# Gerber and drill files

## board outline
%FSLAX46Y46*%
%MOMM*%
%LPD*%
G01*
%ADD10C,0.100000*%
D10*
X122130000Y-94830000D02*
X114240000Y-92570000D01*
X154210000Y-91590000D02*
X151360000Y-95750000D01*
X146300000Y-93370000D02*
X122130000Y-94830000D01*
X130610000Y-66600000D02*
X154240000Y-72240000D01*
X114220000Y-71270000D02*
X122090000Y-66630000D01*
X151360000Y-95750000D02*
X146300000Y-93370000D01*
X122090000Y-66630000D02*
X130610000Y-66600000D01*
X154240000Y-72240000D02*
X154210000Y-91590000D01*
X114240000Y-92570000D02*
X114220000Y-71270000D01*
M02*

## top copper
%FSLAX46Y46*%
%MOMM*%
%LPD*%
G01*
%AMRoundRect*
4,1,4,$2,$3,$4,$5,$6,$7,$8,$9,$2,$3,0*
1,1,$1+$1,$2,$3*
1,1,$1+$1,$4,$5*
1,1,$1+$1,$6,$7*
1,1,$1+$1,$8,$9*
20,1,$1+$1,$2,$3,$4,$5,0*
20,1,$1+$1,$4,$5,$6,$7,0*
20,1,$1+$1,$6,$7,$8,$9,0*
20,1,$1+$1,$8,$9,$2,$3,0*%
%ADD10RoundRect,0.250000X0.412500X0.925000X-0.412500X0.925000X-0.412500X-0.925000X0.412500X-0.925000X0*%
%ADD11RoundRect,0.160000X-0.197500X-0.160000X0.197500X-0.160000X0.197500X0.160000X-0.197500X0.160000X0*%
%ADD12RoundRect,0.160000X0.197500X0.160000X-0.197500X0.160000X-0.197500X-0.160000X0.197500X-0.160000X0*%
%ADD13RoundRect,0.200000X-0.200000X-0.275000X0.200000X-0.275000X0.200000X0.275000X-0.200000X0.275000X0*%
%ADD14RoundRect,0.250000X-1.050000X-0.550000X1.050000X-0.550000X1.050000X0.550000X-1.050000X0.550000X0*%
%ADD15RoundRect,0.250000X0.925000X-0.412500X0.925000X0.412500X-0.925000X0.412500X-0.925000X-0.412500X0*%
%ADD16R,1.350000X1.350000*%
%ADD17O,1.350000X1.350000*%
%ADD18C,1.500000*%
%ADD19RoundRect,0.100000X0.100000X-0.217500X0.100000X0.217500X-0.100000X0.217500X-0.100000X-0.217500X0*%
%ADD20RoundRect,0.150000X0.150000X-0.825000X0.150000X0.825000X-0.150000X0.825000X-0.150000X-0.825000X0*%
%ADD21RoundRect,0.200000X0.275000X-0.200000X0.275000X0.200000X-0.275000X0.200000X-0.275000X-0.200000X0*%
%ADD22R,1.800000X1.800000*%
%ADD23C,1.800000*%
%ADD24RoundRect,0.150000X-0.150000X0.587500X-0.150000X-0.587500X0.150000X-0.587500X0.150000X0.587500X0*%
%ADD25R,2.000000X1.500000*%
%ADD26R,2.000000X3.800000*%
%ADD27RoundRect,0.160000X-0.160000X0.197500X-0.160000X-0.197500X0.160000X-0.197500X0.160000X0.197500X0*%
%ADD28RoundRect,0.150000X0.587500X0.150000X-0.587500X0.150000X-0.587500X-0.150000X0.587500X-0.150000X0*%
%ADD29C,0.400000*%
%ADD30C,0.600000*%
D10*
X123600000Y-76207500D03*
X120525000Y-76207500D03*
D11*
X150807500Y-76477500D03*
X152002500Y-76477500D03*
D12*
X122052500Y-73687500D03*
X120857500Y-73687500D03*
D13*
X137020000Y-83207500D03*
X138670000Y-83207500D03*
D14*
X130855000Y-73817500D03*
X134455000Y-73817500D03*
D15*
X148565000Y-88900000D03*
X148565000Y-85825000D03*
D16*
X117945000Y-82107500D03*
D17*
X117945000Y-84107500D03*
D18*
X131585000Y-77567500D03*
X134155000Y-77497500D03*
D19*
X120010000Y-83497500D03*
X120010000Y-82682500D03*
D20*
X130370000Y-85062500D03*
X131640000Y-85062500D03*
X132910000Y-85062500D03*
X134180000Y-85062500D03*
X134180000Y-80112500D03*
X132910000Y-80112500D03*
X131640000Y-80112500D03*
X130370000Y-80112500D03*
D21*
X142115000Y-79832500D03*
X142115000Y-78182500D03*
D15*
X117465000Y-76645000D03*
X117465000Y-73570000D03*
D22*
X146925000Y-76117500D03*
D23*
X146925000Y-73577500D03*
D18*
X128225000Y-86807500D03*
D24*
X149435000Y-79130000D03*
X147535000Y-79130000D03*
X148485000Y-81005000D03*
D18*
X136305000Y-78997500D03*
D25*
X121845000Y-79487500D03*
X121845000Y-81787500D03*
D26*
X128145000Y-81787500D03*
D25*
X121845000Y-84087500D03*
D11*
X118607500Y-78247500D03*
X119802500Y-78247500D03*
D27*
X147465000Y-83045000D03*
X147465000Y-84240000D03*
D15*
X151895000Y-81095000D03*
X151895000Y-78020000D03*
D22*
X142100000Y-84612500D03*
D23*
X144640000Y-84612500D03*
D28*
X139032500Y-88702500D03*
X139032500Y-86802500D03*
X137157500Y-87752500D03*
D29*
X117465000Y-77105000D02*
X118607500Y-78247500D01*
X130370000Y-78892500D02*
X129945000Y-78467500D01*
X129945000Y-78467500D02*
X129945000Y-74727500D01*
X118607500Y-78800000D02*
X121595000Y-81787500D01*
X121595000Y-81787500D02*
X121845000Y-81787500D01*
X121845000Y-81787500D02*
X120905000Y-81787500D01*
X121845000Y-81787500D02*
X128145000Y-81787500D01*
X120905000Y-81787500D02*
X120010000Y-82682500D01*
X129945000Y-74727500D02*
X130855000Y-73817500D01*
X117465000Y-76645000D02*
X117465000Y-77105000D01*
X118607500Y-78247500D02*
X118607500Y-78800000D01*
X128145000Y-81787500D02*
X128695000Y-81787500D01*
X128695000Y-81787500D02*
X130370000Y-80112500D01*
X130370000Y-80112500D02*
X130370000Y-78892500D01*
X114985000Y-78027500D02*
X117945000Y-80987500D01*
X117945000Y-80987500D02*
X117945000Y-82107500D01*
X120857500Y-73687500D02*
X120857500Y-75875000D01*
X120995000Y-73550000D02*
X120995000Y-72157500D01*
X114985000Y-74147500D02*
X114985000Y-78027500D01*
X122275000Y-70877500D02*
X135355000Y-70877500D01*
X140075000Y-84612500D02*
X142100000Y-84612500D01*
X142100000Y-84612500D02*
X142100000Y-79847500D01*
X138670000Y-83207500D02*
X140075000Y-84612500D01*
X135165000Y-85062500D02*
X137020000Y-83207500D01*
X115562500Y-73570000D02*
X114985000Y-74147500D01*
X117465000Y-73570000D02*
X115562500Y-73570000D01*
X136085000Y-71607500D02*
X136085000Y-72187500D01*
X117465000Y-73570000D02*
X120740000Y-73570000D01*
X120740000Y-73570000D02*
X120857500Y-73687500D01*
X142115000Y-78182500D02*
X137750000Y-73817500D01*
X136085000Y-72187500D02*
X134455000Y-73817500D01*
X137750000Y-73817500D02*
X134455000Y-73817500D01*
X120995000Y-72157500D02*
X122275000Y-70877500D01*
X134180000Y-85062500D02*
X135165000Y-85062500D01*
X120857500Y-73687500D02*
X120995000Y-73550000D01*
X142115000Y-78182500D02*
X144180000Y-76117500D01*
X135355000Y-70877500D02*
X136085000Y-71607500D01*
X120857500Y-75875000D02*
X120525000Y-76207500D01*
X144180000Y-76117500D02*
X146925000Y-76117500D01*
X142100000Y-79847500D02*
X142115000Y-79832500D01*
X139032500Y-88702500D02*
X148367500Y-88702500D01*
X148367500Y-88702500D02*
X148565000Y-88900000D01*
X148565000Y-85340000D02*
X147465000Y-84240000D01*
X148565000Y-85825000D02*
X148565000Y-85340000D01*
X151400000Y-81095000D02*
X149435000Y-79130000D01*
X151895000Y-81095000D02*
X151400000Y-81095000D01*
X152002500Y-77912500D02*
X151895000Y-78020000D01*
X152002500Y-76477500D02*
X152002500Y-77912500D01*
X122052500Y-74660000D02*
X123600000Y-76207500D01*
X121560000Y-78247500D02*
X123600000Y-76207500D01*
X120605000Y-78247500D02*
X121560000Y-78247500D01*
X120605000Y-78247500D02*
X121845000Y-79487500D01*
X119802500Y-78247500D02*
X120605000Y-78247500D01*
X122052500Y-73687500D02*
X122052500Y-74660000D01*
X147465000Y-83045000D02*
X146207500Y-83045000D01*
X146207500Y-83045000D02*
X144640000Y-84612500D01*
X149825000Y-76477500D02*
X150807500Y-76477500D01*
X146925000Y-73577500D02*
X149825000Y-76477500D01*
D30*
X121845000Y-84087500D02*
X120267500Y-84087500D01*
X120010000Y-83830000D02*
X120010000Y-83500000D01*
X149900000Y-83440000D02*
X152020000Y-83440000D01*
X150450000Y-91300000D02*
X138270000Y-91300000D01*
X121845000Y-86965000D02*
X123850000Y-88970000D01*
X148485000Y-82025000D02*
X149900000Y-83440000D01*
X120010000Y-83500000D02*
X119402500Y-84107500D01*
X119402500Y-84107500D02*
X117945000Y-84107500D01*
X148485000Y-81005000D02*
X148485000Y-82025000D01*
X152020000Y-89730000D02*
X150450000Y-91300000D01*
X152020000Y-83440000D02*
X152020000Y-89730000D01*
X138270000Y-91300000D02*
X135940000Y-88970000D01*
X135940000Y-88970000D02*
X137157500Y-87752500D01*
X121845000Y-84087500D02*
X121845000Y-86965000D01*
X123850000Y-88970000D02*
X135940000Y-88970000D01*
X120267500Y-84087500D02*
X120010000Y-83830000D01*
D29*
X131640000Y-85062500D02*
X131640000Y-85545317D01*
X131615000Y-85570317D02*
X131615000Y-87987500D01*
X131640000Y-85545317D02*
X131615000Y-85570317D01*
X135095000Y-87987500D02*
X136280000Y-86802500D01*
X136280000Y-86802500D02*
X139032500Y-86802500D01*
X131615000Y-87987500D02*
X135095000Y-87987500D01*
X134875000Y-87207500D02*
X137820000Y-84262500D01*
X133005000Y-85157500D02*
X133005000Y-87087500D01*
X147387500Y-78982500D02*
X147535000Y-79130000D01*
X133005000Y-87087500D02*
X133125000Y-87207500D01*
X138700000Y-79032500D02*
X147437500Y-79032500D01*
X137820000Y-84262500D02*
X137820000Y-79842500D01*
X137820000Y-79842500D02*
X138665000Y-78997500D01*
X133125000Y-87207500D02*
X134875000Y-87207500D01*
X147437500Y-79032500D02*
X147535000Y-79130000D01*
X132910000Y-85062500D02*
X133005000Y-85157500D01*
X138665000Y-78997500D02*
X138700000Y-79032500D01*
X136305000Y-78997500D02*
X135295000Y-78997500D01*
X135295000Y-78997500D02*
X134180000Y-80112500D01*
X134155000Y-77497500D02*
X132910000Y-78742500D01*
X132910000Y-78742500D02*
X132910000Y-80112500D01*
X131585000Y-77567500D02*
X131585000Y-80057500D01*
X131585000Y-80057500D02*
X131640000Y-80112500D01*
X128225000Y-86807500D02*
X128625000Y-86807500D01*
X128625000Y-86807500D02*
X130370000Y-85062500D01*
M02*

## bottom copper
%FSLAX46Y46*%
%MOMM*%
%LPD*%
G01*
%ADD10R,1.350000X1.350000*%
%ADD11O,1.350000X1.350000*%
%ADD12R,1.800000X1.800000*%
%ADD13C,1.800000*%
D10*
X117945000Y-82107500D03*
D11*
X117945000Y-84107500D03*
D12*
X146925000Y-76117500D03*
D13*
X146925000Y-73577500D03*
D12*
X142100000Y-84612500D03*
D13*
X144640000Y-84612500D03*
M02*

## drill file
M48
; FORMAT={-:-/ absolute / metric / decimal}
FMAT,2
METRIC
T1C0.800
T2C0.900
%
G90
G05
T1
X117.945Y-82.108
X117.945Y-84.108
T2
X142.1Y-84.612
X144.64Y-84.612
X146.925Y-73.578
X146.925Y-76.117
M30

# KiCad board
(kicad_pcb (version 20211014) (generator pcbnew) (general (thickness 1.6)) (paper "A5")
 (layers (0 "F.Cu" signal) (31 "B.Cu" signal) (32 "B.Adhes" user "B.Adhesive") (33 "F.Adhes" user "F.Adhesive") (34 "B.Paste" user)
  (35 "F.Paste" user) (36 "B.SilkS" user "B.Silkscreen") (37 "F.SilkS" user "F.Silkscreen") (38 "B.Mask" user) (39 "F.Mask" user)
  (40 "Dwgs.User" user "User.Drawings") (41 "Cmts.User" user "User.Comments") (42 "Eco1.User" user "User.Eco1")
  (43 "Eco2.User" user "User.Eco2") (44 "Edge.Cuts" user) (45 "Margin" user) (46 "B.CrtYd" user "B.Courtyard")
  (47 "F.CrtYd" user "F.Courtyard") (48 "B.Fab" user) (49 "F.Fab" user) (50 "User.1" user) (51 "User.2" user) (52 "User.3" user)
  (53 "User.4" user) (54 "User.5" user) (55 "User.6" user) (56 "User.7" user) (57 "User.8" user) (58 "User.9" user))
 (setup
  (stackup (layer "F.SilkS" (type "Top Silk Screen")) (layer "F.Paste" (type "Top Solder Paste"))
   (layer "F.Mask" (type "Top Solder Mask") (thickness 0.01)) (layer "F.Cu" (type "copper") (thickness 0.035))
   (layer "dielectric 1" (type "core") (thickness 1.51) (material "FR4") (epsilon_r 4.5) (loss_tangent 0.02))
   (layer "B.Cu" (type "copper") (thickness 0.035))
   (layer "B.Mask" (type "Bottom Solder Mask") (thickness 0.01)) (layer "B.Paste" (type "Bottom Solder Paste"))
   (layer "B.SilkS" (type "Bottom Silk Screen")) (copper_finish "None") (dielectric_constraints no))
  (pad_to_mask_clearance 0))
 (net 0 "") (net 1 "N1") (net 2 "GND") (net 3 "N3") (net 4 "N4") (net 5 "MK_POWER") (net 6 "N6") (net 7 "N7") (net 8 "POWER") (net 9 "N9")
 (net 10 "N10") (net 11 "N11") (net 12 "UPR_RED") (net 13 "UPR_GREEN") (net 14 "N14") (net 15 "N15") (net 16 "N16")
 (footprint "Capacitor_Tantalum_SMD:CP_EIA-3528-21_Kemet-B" (layer "F.Cu") (at 122.0625 76.2075 180)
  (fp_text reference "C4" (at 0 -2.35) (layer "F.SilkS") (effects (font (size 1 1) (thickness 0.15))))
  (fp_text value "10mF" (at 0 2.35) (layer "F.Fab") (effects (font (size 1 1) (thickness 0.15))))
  (pad "1" smd roundrect (at -1.5375 0 180) (size 1.325 2.35) (layers "F.Cu" "F.Paste" "F.Mask") (roundrect_rratio 0.188679) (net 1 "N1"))
  (pad "2" smd roundrect (at 1.5375 0 180) (size 1.325 2.35) (layers "F.Cu" "F.Paste" "F.Mask") (roundrect_rratio 0.188679) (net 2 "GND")))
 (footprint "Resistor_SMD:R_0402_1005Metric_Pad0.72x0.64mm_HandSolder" (layer "F.Cu") (at 151.405 76.4775)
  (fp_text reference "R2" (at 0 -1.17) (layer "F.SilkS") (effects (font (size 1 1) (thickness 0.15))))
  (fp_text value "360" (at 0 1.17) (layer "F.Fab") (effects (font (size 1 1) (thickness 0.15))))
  (pad "1" smd roundrect (at -0.5975 0) (size 0.715 0.64) (layers "F.Cu" "F.Paste" "F.Mask") (roundrect_rratio 0.25) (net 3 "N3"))
  (pad "2" smd roundrect (at 0.5975 0) (size 0.715 0.64) (layers "F.Cu" "F.Paste" "F.Mask") (roundrect_rratio 0.25) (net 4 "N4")))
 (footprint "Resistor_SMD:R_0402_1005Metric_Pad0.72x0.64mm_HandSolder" (layer "F.Cu") (at 121.455 73.6875 180)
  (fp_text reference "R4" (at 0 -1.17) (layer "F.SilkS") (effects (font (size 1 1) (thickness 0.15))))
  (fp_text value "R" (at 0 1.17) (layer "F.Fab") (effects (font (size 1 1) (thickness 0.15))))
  (pad "1" smd roundrect (at -0.5975 0 180) (size 0.715 0.64) (layers "F.Cu" "F.Paste" "F.Mask") (roundrect_rratio 0.25) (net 1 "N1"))
  (pad "2" smd roundrect (at 0.5975 0 180) (size 0.715 0.64) (layers "F.Cu" "F.Paste" "F.Mask") (roundrect_rratio 0.25) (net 2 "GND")))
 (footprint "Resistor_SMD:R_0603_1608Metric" (layer "F.Cu") (at 137.845 83.2075)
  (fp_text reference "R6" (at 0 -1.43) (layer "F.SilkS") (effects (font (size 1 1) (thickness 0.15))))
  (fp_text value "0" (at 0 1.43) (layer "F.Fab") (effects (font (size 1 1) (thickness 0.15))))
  (pad "1" smd roundrect (at -0.825 0) (size 0.8 0.95) (layers "F.Cu" "F.Paste" "F.Mask") (roundrect_rratio 0.25) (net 2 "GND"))
  (pad "2" smd roundrect (at 0.825 0) (size 0.8 0.95) (layers "F.Cu" "F.Paste" "F.Mask") (roundrect_rratio 0.25) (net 2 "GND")))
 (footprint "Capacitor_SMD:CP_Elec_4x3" (layer "F.Cu") (at 132.655 73.8175)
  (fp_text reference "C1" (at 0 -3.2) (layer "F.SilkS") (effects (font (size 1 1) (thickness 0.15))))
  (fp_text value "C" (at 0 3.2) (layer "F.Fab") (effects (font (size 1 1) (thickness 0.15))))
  (pad "1" smd roundrect (at -1.8 0) (size 2.6 1.6) (layers "F.Cu" "F.Paste" "F.Mask") (roundrect_rratio 0.15625) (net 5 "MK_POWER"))
  (pad "2" smd roundrect (at 1.8 0) (size 2.6 1.6) (layers "F.Cu" "F.Paste" "F.Mask") (roundrect_rratio 0.15625) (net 2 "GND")))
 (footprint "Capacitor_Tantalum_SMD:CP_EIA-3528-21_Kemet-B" (layer "F.Cu") (at 148.565 87.3625 90)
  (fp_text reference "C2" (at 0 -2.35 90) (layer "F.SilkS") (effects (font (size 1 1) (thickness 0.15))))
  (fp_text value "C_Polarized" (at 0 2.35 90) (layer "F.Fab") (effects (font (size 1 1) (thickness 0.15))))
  (pad "1" smd roundrect (at -1.5375 0 90) (size 1.325 2.35) (layers "F.Cu" "F.Paste" "F.Mask") (roundrect_rratio 0.188679) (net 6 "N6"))
  (pad "2" smd roundrect (at 1.5375 0 90) (size 1.325 2.35) (layers "F.Cu" "F.Paste" "F.Mask") (roundrect_rratio 0.188679) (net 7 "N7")))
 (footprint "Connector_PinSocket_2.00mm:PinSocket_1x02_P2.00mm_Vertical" (layer "F.Cu") (at 117.945 82.1075)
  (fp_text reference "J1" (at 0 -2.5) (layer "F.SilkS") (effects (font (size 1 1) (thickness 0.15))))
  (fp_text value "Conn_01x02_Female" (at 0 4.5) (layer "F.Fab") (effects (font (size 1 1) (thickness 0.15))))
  (pad "1" thru_hole rect (at 0 0) (size 1.35 1.35) (drill 0.8) (layers *.Cu *.Mask) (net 2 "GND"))
  (pad "2" thru_hole oval (at 0 2) (size 1.35 1.35) (drill 0.8) (layers *.Cu *.Mask) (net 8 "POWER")))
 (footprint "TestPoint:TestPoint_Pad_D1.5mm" (layer "F.Cu") (at 131.585 77.5675)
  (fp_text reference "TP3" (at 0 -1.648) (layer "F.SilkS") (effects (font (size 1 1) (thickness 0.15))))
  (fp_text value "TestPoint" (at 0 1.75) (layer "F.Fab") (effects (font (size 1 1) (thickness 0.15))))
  (pad "1" smd circle (at 0 0) (size 1.5 1.5) (layers "F.Cu" "F.Mask") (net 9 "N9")))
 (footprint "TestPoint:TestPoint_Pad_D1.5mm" (layer "F.Cu") (at 134.155 77.4975)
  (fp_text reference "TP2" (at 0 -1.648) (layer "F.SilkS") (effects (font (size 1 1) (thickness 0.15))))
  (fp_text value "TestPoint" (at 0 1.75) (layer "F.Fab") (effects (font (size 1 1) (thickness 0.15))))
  (pad "1" smd circle (at 0 0) (size 1.5 1.5) (layers "F.Cu" "F.Mask") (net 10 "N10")))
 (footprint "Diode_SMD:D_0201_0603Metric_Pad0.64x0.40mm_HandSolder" (layer "F.Cu") (at 120.01 83.09 90)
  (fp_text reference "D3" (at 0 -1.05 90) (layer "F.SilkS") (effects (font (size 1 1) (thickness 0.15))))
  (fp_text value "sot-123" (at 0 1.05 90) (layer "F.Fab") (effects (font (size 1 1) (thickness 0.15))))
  (pad "" smd roundrect (at 0.4325 0 90) (size 0.458 0.36) (layers "F.Paste") (roundrect_rratio 0.25))
  (pad "" smd roundrect (at -0.4325 0 90) (size 0.458 0.36) (layers "F.Paste") (roundrect_rratio 0.25))
  (pad "1" smd roundrect (at -0.4075 0 90) (size 0.635 0.4) (layers "F.Cu" "F.Mask") (roundrect_rratio 0.25) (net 8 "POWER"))
  (pad "2" smd roundrect (at 0.4075 0 90) (size 0.635 0.4) (layers "F.Cu" "F.Mask") (roundrect_rratio 0.25) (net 5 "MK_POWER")))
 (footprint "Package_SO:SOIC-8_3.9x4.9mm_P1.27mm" (layer "F.Cu") (at 132.275 82.5875 90)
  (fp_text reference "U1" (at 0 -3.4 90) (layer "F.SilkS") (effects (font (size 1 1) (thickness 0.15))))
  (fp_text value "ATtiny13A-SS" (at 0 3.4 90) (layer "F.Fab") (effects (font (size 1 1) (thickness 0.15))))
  (pad "1" smd roundrect (at -2.475 -1.905 90) (size 1.95 0.6) (layers "F.Cu" "F.Paste" "F.Mask") (roundrect_rratio 0.25) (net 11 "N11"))
  (pad "2" smd roundrect (at -2.475 -0.635 90) (size 1.95 0.6) (layers "F.Cu" "F.Paste" "F.Mask") (roundrect_rratio 0.25) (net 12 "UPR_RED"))
  (pad "3" smd roundrect (at -2.475 0.635 90) (size 1.95 0.6) (layers "F.Cu" "F.Paste" "F.Mask") (roundrect_rratio 0.25)
   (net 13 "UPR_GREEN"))
  (pad "4" smd roundrect (at -2.475 1.905 90) (size 1.95 0.6) (layers "F.Cu" "F.Paste" "F.Mask") (roundrect_rratio 0.25) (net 2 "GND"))
  (pad "5" smd roundrect (at 2.475 1.905 90) (size 1.95 0.6) (layers "F.Cu" "F.Paste" "F.Mask") (roundrect_rratio 0.25) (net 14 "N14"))
  (pad "6" smd roundrect (at 2.475 0.635 90) (size 1.95 0.6) (layers "F.Cu" "F.Paste" "F.Mask") (roundrect_rratio 0.25) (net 10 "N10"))
  (pad "7" smd roundrect (at 2.475 -0.635 90) (size 1.95 0.6) (layers "F.Cu" "F.Paste" "F.Mask") (roundrect_rratio 0.25) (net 9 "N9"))
  (pad "8" smd roundrect (at 2.475 -1.905 90) (size 1.95 0.6) (layers "F.Cu" "F.Paste" "F.Mask") (roundrect_rratio 0.25) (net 5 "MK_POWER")))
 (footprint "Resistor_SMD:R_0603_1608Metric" (layer "F.Cu") (at 142.115 79.0075 90)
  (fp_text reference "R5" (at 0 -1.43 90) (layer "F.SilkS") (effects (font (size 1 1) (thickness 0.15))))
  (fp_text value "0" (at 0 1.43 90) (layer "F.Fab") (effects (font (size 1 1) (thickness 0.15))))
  (pad "1" smd roundrect (at -0.825 0 90) (size 0.8 0.95) (layers "F.Cu" "F.Paste" "F.Mask") (roundrect_rratio 0.25) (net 2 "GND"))
  (pad "2" smd roundrect (at 0.825 0 90) (size 0.8 0.95) (layers "F.Cu" "F.Paste" "F.Mask") (roundrect_rratio 0.25) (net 2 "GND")))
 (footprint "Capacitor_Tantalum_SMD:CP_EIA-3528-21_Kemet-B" (layer "F.Cu") (at 117.465 75.1075 90)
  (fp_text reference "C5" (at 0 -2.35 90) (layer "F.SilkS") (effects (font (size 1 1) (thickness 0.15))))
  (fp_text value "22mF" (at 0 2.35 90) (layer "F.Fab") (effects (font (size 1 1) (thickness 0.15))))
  (pad "1" smd roundrect (at -1.5375 0 90) (size 1.325 2.35) (layers "F.Cu" "F.Paste" "F.Mask") (roundrect_rratio 0.188679)
   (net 5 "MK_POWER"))
  (pad "2" smd roundrect (at 1.5375 0 90) (size 1.325 2.35) (layers "F.Cu" "F.Paste" "F.Mask") (roundrect_rratio 0.188679) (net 2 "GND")))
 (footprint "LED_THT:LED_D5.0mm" (layer "F.Cu") (at 146.925 76.1175 90)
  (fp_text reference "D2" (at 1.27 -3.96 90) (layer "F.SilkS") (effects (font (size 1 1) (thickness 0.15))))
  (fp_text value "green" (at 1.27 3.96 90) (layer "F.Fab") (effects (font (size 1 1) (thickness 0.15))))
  (pad "1" thru_hole rect (at 0 0 90) (size 1.8 1.8) (drill 0.9) (layers *.Cu *.Mask) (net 2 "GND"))
  (pad "2" thru_hole circle (at 2.54 0 90) (size 1.8 1.8) (drill 0.9) (layers *.Cu *.Mask) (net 3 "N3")))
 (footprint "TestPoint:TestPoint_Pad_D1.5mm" (layer "F.Cu") (at 128.225 86.8075)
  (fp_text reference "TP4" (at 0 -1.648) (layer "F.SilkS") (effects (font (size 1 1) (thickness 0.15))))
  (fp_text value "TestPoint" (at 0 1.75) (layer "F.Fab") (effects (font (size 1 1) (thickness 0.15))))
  (pad "1" smd circle (at 0 0) (size 1.5 1.5) (layers "F.Cu" "F.Mask") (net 11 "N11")))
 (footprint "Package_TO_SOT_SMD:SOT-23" (layer "F.Cu") (at 148.485 80.0675 -90)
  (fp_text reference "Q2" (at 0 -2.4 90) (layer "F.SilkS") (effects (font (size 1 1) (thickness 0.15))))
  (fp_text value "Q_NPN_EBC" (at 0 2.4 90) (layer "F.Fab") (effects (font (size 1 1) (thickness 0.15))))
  (pad "1" smd roundrect (at -0.9375 -0.95 270) (size 1.475 0.6) (layers "F.Cu" "F.Paste" "F.Mask") (roundrect_rratio 0.25) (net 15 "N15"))
  (pad "2" smd roundrect (at -0.9375 0.95 270) (size 1.475 0.6) (layers "F.Cu" "F.Paste" "F.Mask") (roundrect_rratio 0.25)
   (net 13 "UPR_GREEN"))
  (pad "3" smd roundrect (at 0.9375 0 270) (size 1.475 0.6) (layers "F.Cu" "F.Paste" "F.Mask") (roundrect_rratio 0.25) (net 8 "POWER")))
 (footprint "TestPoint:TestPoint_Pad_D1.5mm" (layer "F.Cu") (at 136.305 78.9975)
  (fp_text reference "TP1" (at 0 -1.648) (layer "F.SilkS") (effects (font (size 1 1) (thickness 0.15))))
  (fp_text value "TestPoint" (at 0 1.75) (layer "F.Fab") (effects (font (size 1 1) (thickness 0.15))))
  (pad "1" smd circle (at 0 0) (size 1.5 1.5) (layers "F.Cu" "F.Mask") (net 14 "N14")))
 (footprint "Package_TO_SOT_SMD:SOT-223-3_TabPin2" (layer "F.Cu") (at 124.995 81.7875)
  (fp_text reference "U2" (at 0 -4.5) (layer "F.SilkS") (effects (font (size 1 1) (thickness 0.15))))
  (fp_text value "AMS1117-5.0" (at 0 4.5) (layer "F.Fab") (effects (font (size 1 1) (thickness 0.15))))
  (pad "1" smd rect (at -3.15 -2.3) (size 2 1.5) (layers "F.Cu" "F.Paste" "F.Mask") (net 1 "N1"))
  (pad "2" smd rect (at -3.15 0) (size 2 1.5) (layers "F.Cu" "F.Paste" "F.Mask") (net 5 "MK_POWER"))
  (pad "2" smd rect (at 3.15 0) (size 2 3.8) (layers "F.Cu" "F.Paste" "F.Mask") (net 5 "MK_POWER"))
  (pad "3" smd rect (at -3.15 2.3) (size 2 1.5) (layers "F.Cu" "F.Paste" "F.Mask") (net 8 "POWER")))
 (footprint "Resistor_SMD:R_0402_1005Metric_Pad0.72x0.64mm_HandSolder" (layer "F.Cu") (at 119.205 78.2475)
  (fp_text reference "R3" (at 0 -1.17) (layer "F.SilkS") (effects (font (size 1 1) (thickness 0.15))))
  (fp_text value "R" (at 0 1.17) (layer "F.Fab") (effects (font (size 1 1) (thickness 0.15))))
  (pad "1" smd roundrect (at -0.5975 0) (size 0.715 0.64) (layers "F.Cu" "F.Paste" "F.Mask") (roundrect_rratio 0.25) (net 5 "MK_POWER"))
  (pad "2" smd roundrect (at 0.5975 0) (size 0.715 0.64) (layers "F.Cu" "F.Paste" "F.Mask") (roundrect_rratio 0.25) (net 1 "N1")))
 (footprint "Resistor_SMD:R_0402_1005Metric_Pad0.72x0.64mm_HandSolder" (layer "F.Cu") (at 147.465 83.6425 -90)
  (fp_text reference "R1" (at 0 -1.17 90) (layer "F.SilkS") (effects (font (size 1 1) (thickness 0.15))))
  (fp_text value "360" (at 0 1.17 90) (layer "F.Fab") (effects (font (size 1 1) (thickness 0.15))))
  (pad "1" smd roundrect (at -0.5975 0 270) (size 0.715 0.64) (layers "F.Cu" "F.Paste" "F.Mask") (roundrect_rratio 0.25) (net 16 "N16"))
  (pad "2" smd roundrect (at 0.5975 0 270) (size 0.715 0.64) (layers "F.Cu" "F.Paste" "F.Mask") (roundrect_rratio 0.25) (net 7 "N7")))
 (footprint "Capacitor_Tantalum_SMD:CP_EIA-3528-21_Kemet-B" (layer "F.Cu") (at 151.895 79.5575 90)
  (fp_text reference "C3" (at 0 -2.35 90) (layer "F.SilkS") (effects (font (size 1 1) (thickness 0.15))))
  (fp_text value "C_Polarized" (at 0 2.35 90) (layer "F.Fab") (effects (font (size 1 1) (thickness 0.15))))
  (pad "1" smd roundrect (at -1.5375 0 90) (size 1.325 2.35) (layers "F.Cu" "F.Paste" "F.Mask") (roundrect_rratio 0.188679) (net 15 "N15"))
  (pad "2" smd roundrect (at 1.5375 0 90) (size 1.325 2.35) (layers "F.Cu" "F.Paste" "F.Mask") (roundrect_rratio 0.188679) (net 4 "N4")))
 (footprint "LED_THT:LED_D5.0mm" (layer "F.Cu") (at 142.1 84.6125)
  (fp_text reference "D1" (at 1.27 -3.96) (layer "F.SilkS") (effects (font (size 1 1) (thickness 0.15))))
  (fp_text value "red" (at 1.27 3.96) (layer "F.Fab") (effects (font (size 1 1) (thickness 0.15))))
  (pad "1" thru_hole rect (at 0 0) (size 1.8 1.8) (drill 0.9) (layers *.Cu *.Mask) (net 2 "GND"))
  (pad "2" thru_hole circle (at 2.54 0) (size 1.8 1.8) (drill 0.9) (layers *.Cu *.Mask) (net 16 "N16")))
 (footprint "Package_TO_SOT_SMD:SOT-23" (layer "F.Cu") (at 138.095 87.7525 180)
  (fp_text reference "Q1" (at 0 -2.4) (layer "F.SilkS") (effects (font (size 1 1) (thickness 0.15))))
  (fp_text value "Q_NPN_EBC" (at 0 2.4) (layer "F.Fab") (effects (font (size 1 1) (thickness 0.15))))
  (pad "1" smd roundrect (at -0.9375 -0.95 180) (size 1.475 0.6) (layers "F.Cu" "F.Paste" "F.Mask") (roundrect_rratio 0.25) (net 6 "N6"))
  (pad "2" smd roundrect (at -0.9375 0.95 180) (size 1.475 0.6) (layers "F.Cu" "F.Paste" "F.Mask") (roundrect_rratio 0.25)
   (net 12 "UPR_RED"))
  (pad "3" smd roundrect (at 0.9375 0 180) (size 1.475 0.6) (layers "F.Cu" "F.Paste" "F.Mask") (roundrect_rratio 0.25) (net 8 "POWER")))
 (gr_line (start 122.13 94.83) (end 114.24 92.57) (layer "Edge.Cuts") (width 0.1))
 (gr_line (start 154.21 91.59) (end 151.36 95.75) (layer "Edge.Cuts") (width 0.1))
 (gr_line (start 146.3 93.37) (end 122.13 94.83) (layer "Edge.Cuts") (width 0.1))
 (gr_line (start 130.61 66.6) (end 154.24 72.24) (layer "Edge.Cuts") (width 0.1))
 (gr_line (start 114.22 71.27) (end 122.09 66.63) (layer "Edge.Cuts") (width 0.1))
 (gr_line (start 151.36 95.75) (end 146.3 93.37) (layer "Edge.Cuts") (width 0.1))
 (gr_line (start 122.09 66.63) (end 130.61 66.6) (layer "Edge.Cuts") (width 0.1))
 (gr_line (start 154.24 72.24) (end 154.21 91.59) (layer "Edge.Cuts") (width 0.1))
 (gr_line (start 114.24 92.57) (end 114.22 71.27) (layer "Edge.Cuts") (width 0.1))
 (segment (start 117.465 77.105) (end 118.6075 78.2475) (width 0.4) (layer "F.Cu") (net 5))
 (segment (start 130.37 78.8925) (end 129.945 78.4675) (width 0.4) (layer "F.Cu") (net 5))
 (segment (start 129.945 78.4675) (end 129.945 74.7275) (width 0.4) (layer "F.Cu") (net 5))
 (segment (start 118.6075 78.8) (end 121.595 81.7875) (width 0.4) (layer "F.Cu") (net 5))
 (segment (start 121.595 81.7875) (end 121.845 81.7875) (width 0.4) (layer "F.Cu") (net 5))
 (segment (start 121.845 81.7875) (end 120.905 81.7875) (width 0.4) (layer "F.Cu") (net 5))
 (segment (start 121.845 81.7875) (end 128.145 81.7875) (width 0.4) (layer "F.Cu") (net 5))
 (segment (start 120.905 81.7875) (end 120.01 82.6825) (width 0.4) (layer "F.Cu") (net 5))
 (segment (start 129.945 74.7275) (end 130.855 73.8175) (width 0.4) (layer "F.Cu") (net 5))
 (segment (start 117.465 76.645) (end 117.465 77.105) (width 0.4) (layer "F.Cu") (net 5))
 (segment (start 118.6075 78.2475) (end 118.6075 78.8) (width 0.4) (layer "F.Cu") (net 5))
 (segment (start 128.145 81.7875) (end 128.695 81.7875) (width 0.4) (layer "F.Cu") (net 5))
 (segment (start 128.695 81.7875) (end 130.37 80.1125) (width 0.4) (layer "F.Cu") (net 5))
 (segment (start 130.37 80.1125) (end 130.37 78.8925) (width 0.4) (layer "F.Cu") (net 5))
 (segment (start 114.985 78.0275) (end 117.945 80.9875) (width 0.4) (layer "F.Cu") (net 2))
 (segment (start 117.945 80.9875) (end 117.945 82.1075) (width 0.4) (layer "F.Cu") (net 2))
 (segment (start 120.8575 73.6875) (end 120.8575 75.875) (width 0.4) (layer "F.Cu") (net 2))
 (segment (start 120.995 73.55) (end 120.995 72.1575) (width 0.4) (layer "F.Cu") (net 2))
 (segment (start 114.985 74.1475) (end 114.985 78.0275) (width 0.4) (layer "F.Cu") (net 2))
 (segment (start 122.275 70.8775) (end 135.355 70.8775) (width 0.4) (layer "F.Cu") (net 2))
 (segment (start 140.075 84.6125) (end 142.1 84.6125) (width 0.4) (layer "F.Cu") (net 2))
 (segment (start 142.1 84.6125) (end 142.1 79.8475) (width 0.4) (layer "F.Cu") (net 2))
 (segment (start 138.67 83.2075) (end 140.075 84.6125) (width 0.4) (layer "F.Cu") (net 2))
 (segment (start 135.165 85.0625) (end 137.02 83.2075) (width 0.4) (layer "F.Cu") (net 2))
 (segment (start 115.5625 73.57) (end 114.985 74.1475) (width 0.4) (layer "F.Cu") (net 2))
 (segment (start 117.465 73.57) (end 115.5625 73.57) (width 0.4) (layer "F.Cu") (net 2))
 (segment (start 136.085 71.6075) (end 136.085 72.1875) (width 0.4) (layer "F.Cu") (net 2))
 (segment (start 117.465 73.57) (end 120.74 73.57) (width 0.4) (layer "F.Cu") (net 2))
 (segment (start 120.74 73.57) (end 120.8575 73.6875) (width 0.4) (layer "F.Cu") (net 2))
 (segment (start 142.115 78.1825) (end 137.75 73.8175) (width 0.4) (layer "F.Cu") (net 2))
 (segment (start 136.085 72.1875) (end 134.455 73.8175) (width 0.4) (layer "F.Cu") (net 2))
 (segment (start 137.75 73.8175) (end 134.455 73.8175) (width 0.4) (layer "F.Cu") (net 2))
 (segment (start 120.995 72.1575) (end 122.275 70.8775) (width 0.4) (layer "F.Cu") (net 2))
 (segment (start 134.18 85.0625) (end 135.165 85.0625) (width 0.4) (layer "F.Cu") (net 2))
 (segment (start 120.8575 73.6875) (end 120.995 73.55) (width 0.4) (layer "F.Cu") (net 2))
 (segment (start 142.115 78.1825) (end 144.18 76.1175) (width 0.4) (layer "F.Cu") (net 2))
 (segment (start 135.355 70.8775) (end 136.085 71.6075) (width 0.4) (layer "F.Cu") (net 2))
 (segment (start 120.8575 75.875) (end 120.525 76.2075) (width 0.4) (layer "F.Cu") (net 2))
 (segment (start 144.18 76.1175) (end 146.925 76.1175) (width 0.4) (layer "F.Cu") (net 2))
 (segment (start 142.1 79.8475) (end 142.115 79.8325) (width 0.4) (layer "F.Cu") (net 2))
 (segment (start 139.0325 88.7025) (end 148.3675 88.7025) (width 0.4) (layer "F.Cu") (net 6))
 (segment (start 148.3675 88.7025) (end 148.565 88.9) (width 0.4) (layer "F.Cu") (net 6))
 (segment (start 148.565 85.34) (end 147.465 84.24) (width 0.4) (layer "F.Cu") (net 7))
 (segment (start 148.565 85.825) (end 148.565 85.34) (width 0.4) (layer "F.Cu") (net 7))
 (segment (start 151.4 81.095) (end 149.435 79.13) (width 0.4) (layer "F.Cu") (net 15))
 (segment (start 151.895 81.095) (end 151.4 81.095) (width 0.4) (layer "F.Cu") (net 15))
 (segment (start 152.0025 77.9125) (end 151.895 78.02) (width 0.4) (layer "F.Cu") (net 4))
 (segment (start 152.0025 76.4775) (end 152.0025 77.9125) (width 0.4) (layer "F.Cu") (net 4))
 (segment (start 122.0525 74.66) (end 123.6 76.2075) (width 0.4) (layer "F.Cu") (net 1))
 (segment (start 121.56 78.2475) (end 123.6 76.2075) (width 0.4) (layer "F.Cu") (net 1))
 (segment (start 120.605 78.2475) (end 121.56 78.2475) (width 0.4) (layer "F.Cu") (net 1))
 (segment (start 120.605 78.2475) (end 121.845 79.4875) (width 0.4) (layer "F.Cu") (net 1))
 (segment (start 119.8025 78.2475) (end 120.605 78.2475) (width 0.4) (layer "F.Cu") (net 1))
 (segment (start 122.0525 73.6875) (end 122.0525 74.66) (width 0.4) (layer "F.Cu") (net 1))
 (segment (start 147.465 83.045) (end 146.2075 83.045) (width 0.4) (layer "F.Cu") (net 16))
 (segment (start 146.2075 83.045) (end 144.64 84.6125) (width 0.4) (layer "F.Cu") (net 16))
 (segment (start 149.825 76.4775) (end 150.8075 76.4775) (width 0.4) (layer "F.Cu") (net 3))
 (segment (start 146.925 73.5775) (end 149.825 76.4775) (width 0.4) (layer "F.Cu") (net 3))
 (segment (start 121.845 84.0875) (end 120.2675 84.0875) (width 0.6) (layer "F.Cu") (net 8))
 (segment (start 120.01 83.83) (end 120.01 83.5) (width 0.6) (layer "F.Cu") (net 8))
 (segment (start 149.9 83.44) (end 152.02 83.44) (width 0.6) (layer "F.Cu") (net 8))
 (segment (start 150.45 91.3) (end 138.27 91.3) (width 0.6) (layer "F.Cu") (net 8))
 (segment (start 121.845 86.965) (end 123.85 88.97) (width 0.6) (layer "F.Cu") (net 8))
 (segment (start 148.485 82.025) (end 149.9 83.44) (width 0.6) (layer "F.Cu") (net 8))
 (segment (start 120.01 83.5) (end 119.4025 84.1075) (width 0.6) (layer "F.Cu") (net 8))
 (segment (start 119.4025 84.1075) (end 117.945 84.1075) (width 0.6) (layer "F.Cu") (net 8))
 (segment (start 148.485 81.005) (end 148.485 82.025) (width 0.6) (layer "F.Cu") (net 8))
 (segment (start 152.02 89.73) (end 150.45 91.3) (width 0.6) (layer "F.Cu") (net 8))
 (segment (start 152.02 83.44) (end 152.02 89.73) (width 0.6) (layer "F.Cu") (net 8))
 (segment (start 138.27 91.3) (end 135.94 88.97) (width 0.6) (layer "F.Cu") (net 8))
 (segment (start 135.94 88.97) (end 137.1575 87.7525) (width 0.6) (layer "F.Cu") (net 8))
 (segment (start 121.845 84.0875) (end 121.845 86.965) (width 0.6) (layer "F.Cu") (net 8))
 (segment (start 123.85 88.97) (end 135.94 88.97) (width 0.6) (layer "F.Cu") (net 8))
 (segment (start 120.2675 84.0875) (end 120.01 83.83) (width 0.6) (layer "F.Cu") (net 8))
 (segment (start 131.64 85.0625) (end 131.64 85.545317) (width 0.4) (layer "F.Cu") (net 12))
 (segment (start 131.615 85.570317) (end 131.615 87.9875) (width 0.4) (layer "F.Cu") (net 12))
 (segment (start 131.64 85.545317) (end 131.615 85.570317) (width 0.4) (layer "F.Cu") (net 12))
 (segment (start 135.095 87.9875) (end 136.28 86.8025) (width 0.4) (layer "F.Cu") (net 12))
 (segment (start 136.28 86.8025) (end 139.0325 86.8025) (width 0.4) (layer "F.Cu") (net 12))
 (segment (start 131.615 87.9875) (end 135.095 87.9875) (width 0.4) (layer "F.Cu") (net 12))
 (segment (start 134.875 87.2075) (end 137.82 84.2625) (width 0.4) (layer "F.Cu") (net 13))
 (segment (start 133.005 85.1575) (end 133.005 87.0875) (width 0.4) (layer "F.Cu") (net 13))
 (segment (start 147.3875 78.9825) (end 147.535 79.13) (width 0.4) (layer "F.Cu") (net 13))
 (segment (start 133.005 87.0875) (end 133.125 87.2075) (width 0.4) (layer "F.Cu") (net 13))
 (segment (start 138.7 79.0325) (end 147.4375 79.0325) (width 0.4) (layer "F.Cu") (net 13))
 (segment (start 137.82 84.2625) (end 137.82 79.8425) (width 0.4) (layer "F.Cu") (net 13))
 (segment (start 137.82 79.8425) (end 138.665 78.9975) (width 0.4) (layer "F.Cu") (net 13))
 (segment (start 133.125 87.2075) (end 134.875 87.2075) (width 0.4) (layer "F.Cu") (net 13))
 (segment (start 147.4375 79.0325) (end 147.535 79.13) (width 0.4) (layer "F.Cu") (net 13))
 (segment (start 132.91 85.0625) (end 133.005 85.1575) (width 0.4) (layer "F.Cu") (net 13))
 (segment (start 138.665 78.9975) (end 138.7 79.0325) (width 0.4) (layer "F.Cu") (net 13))
 (segment (start 136.305 78.9975) (end 135.295 78.9975) (width 0.4) (layer "F.Cu") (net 14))
 (segment (start 135.295 78.9975) (end 134.18 80.1125) (width 0.4) (layer "F.Cu") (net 14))
 (segment (start 134.155 77.4975) (end 132.91 78.7425) (width 0.4) (layer "F.Cu") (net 10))
 (segment (start 132.91 78.7425) (end 132.91 80.1125) (width 0.4) (layer "F.Cu") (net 10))
 (segment (start 131.585 77.5675) (end 131.585 80.0575) (width 0.4) (layer "F.Cu") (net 9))
 (segment (start 131.585 80.0575) (end 131.64 80.1125) (width 0.4) (layer "F.Cu") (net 9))
 (segment (start 128.225 86.8075) (end 128.625 86.8075) (width 0.4) (layer "F.Cu") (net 11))
 (segment (start 128.625 86.8075) (end 130.37 85.0625) (width 0.4) (layer "F.Cu") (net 11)))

